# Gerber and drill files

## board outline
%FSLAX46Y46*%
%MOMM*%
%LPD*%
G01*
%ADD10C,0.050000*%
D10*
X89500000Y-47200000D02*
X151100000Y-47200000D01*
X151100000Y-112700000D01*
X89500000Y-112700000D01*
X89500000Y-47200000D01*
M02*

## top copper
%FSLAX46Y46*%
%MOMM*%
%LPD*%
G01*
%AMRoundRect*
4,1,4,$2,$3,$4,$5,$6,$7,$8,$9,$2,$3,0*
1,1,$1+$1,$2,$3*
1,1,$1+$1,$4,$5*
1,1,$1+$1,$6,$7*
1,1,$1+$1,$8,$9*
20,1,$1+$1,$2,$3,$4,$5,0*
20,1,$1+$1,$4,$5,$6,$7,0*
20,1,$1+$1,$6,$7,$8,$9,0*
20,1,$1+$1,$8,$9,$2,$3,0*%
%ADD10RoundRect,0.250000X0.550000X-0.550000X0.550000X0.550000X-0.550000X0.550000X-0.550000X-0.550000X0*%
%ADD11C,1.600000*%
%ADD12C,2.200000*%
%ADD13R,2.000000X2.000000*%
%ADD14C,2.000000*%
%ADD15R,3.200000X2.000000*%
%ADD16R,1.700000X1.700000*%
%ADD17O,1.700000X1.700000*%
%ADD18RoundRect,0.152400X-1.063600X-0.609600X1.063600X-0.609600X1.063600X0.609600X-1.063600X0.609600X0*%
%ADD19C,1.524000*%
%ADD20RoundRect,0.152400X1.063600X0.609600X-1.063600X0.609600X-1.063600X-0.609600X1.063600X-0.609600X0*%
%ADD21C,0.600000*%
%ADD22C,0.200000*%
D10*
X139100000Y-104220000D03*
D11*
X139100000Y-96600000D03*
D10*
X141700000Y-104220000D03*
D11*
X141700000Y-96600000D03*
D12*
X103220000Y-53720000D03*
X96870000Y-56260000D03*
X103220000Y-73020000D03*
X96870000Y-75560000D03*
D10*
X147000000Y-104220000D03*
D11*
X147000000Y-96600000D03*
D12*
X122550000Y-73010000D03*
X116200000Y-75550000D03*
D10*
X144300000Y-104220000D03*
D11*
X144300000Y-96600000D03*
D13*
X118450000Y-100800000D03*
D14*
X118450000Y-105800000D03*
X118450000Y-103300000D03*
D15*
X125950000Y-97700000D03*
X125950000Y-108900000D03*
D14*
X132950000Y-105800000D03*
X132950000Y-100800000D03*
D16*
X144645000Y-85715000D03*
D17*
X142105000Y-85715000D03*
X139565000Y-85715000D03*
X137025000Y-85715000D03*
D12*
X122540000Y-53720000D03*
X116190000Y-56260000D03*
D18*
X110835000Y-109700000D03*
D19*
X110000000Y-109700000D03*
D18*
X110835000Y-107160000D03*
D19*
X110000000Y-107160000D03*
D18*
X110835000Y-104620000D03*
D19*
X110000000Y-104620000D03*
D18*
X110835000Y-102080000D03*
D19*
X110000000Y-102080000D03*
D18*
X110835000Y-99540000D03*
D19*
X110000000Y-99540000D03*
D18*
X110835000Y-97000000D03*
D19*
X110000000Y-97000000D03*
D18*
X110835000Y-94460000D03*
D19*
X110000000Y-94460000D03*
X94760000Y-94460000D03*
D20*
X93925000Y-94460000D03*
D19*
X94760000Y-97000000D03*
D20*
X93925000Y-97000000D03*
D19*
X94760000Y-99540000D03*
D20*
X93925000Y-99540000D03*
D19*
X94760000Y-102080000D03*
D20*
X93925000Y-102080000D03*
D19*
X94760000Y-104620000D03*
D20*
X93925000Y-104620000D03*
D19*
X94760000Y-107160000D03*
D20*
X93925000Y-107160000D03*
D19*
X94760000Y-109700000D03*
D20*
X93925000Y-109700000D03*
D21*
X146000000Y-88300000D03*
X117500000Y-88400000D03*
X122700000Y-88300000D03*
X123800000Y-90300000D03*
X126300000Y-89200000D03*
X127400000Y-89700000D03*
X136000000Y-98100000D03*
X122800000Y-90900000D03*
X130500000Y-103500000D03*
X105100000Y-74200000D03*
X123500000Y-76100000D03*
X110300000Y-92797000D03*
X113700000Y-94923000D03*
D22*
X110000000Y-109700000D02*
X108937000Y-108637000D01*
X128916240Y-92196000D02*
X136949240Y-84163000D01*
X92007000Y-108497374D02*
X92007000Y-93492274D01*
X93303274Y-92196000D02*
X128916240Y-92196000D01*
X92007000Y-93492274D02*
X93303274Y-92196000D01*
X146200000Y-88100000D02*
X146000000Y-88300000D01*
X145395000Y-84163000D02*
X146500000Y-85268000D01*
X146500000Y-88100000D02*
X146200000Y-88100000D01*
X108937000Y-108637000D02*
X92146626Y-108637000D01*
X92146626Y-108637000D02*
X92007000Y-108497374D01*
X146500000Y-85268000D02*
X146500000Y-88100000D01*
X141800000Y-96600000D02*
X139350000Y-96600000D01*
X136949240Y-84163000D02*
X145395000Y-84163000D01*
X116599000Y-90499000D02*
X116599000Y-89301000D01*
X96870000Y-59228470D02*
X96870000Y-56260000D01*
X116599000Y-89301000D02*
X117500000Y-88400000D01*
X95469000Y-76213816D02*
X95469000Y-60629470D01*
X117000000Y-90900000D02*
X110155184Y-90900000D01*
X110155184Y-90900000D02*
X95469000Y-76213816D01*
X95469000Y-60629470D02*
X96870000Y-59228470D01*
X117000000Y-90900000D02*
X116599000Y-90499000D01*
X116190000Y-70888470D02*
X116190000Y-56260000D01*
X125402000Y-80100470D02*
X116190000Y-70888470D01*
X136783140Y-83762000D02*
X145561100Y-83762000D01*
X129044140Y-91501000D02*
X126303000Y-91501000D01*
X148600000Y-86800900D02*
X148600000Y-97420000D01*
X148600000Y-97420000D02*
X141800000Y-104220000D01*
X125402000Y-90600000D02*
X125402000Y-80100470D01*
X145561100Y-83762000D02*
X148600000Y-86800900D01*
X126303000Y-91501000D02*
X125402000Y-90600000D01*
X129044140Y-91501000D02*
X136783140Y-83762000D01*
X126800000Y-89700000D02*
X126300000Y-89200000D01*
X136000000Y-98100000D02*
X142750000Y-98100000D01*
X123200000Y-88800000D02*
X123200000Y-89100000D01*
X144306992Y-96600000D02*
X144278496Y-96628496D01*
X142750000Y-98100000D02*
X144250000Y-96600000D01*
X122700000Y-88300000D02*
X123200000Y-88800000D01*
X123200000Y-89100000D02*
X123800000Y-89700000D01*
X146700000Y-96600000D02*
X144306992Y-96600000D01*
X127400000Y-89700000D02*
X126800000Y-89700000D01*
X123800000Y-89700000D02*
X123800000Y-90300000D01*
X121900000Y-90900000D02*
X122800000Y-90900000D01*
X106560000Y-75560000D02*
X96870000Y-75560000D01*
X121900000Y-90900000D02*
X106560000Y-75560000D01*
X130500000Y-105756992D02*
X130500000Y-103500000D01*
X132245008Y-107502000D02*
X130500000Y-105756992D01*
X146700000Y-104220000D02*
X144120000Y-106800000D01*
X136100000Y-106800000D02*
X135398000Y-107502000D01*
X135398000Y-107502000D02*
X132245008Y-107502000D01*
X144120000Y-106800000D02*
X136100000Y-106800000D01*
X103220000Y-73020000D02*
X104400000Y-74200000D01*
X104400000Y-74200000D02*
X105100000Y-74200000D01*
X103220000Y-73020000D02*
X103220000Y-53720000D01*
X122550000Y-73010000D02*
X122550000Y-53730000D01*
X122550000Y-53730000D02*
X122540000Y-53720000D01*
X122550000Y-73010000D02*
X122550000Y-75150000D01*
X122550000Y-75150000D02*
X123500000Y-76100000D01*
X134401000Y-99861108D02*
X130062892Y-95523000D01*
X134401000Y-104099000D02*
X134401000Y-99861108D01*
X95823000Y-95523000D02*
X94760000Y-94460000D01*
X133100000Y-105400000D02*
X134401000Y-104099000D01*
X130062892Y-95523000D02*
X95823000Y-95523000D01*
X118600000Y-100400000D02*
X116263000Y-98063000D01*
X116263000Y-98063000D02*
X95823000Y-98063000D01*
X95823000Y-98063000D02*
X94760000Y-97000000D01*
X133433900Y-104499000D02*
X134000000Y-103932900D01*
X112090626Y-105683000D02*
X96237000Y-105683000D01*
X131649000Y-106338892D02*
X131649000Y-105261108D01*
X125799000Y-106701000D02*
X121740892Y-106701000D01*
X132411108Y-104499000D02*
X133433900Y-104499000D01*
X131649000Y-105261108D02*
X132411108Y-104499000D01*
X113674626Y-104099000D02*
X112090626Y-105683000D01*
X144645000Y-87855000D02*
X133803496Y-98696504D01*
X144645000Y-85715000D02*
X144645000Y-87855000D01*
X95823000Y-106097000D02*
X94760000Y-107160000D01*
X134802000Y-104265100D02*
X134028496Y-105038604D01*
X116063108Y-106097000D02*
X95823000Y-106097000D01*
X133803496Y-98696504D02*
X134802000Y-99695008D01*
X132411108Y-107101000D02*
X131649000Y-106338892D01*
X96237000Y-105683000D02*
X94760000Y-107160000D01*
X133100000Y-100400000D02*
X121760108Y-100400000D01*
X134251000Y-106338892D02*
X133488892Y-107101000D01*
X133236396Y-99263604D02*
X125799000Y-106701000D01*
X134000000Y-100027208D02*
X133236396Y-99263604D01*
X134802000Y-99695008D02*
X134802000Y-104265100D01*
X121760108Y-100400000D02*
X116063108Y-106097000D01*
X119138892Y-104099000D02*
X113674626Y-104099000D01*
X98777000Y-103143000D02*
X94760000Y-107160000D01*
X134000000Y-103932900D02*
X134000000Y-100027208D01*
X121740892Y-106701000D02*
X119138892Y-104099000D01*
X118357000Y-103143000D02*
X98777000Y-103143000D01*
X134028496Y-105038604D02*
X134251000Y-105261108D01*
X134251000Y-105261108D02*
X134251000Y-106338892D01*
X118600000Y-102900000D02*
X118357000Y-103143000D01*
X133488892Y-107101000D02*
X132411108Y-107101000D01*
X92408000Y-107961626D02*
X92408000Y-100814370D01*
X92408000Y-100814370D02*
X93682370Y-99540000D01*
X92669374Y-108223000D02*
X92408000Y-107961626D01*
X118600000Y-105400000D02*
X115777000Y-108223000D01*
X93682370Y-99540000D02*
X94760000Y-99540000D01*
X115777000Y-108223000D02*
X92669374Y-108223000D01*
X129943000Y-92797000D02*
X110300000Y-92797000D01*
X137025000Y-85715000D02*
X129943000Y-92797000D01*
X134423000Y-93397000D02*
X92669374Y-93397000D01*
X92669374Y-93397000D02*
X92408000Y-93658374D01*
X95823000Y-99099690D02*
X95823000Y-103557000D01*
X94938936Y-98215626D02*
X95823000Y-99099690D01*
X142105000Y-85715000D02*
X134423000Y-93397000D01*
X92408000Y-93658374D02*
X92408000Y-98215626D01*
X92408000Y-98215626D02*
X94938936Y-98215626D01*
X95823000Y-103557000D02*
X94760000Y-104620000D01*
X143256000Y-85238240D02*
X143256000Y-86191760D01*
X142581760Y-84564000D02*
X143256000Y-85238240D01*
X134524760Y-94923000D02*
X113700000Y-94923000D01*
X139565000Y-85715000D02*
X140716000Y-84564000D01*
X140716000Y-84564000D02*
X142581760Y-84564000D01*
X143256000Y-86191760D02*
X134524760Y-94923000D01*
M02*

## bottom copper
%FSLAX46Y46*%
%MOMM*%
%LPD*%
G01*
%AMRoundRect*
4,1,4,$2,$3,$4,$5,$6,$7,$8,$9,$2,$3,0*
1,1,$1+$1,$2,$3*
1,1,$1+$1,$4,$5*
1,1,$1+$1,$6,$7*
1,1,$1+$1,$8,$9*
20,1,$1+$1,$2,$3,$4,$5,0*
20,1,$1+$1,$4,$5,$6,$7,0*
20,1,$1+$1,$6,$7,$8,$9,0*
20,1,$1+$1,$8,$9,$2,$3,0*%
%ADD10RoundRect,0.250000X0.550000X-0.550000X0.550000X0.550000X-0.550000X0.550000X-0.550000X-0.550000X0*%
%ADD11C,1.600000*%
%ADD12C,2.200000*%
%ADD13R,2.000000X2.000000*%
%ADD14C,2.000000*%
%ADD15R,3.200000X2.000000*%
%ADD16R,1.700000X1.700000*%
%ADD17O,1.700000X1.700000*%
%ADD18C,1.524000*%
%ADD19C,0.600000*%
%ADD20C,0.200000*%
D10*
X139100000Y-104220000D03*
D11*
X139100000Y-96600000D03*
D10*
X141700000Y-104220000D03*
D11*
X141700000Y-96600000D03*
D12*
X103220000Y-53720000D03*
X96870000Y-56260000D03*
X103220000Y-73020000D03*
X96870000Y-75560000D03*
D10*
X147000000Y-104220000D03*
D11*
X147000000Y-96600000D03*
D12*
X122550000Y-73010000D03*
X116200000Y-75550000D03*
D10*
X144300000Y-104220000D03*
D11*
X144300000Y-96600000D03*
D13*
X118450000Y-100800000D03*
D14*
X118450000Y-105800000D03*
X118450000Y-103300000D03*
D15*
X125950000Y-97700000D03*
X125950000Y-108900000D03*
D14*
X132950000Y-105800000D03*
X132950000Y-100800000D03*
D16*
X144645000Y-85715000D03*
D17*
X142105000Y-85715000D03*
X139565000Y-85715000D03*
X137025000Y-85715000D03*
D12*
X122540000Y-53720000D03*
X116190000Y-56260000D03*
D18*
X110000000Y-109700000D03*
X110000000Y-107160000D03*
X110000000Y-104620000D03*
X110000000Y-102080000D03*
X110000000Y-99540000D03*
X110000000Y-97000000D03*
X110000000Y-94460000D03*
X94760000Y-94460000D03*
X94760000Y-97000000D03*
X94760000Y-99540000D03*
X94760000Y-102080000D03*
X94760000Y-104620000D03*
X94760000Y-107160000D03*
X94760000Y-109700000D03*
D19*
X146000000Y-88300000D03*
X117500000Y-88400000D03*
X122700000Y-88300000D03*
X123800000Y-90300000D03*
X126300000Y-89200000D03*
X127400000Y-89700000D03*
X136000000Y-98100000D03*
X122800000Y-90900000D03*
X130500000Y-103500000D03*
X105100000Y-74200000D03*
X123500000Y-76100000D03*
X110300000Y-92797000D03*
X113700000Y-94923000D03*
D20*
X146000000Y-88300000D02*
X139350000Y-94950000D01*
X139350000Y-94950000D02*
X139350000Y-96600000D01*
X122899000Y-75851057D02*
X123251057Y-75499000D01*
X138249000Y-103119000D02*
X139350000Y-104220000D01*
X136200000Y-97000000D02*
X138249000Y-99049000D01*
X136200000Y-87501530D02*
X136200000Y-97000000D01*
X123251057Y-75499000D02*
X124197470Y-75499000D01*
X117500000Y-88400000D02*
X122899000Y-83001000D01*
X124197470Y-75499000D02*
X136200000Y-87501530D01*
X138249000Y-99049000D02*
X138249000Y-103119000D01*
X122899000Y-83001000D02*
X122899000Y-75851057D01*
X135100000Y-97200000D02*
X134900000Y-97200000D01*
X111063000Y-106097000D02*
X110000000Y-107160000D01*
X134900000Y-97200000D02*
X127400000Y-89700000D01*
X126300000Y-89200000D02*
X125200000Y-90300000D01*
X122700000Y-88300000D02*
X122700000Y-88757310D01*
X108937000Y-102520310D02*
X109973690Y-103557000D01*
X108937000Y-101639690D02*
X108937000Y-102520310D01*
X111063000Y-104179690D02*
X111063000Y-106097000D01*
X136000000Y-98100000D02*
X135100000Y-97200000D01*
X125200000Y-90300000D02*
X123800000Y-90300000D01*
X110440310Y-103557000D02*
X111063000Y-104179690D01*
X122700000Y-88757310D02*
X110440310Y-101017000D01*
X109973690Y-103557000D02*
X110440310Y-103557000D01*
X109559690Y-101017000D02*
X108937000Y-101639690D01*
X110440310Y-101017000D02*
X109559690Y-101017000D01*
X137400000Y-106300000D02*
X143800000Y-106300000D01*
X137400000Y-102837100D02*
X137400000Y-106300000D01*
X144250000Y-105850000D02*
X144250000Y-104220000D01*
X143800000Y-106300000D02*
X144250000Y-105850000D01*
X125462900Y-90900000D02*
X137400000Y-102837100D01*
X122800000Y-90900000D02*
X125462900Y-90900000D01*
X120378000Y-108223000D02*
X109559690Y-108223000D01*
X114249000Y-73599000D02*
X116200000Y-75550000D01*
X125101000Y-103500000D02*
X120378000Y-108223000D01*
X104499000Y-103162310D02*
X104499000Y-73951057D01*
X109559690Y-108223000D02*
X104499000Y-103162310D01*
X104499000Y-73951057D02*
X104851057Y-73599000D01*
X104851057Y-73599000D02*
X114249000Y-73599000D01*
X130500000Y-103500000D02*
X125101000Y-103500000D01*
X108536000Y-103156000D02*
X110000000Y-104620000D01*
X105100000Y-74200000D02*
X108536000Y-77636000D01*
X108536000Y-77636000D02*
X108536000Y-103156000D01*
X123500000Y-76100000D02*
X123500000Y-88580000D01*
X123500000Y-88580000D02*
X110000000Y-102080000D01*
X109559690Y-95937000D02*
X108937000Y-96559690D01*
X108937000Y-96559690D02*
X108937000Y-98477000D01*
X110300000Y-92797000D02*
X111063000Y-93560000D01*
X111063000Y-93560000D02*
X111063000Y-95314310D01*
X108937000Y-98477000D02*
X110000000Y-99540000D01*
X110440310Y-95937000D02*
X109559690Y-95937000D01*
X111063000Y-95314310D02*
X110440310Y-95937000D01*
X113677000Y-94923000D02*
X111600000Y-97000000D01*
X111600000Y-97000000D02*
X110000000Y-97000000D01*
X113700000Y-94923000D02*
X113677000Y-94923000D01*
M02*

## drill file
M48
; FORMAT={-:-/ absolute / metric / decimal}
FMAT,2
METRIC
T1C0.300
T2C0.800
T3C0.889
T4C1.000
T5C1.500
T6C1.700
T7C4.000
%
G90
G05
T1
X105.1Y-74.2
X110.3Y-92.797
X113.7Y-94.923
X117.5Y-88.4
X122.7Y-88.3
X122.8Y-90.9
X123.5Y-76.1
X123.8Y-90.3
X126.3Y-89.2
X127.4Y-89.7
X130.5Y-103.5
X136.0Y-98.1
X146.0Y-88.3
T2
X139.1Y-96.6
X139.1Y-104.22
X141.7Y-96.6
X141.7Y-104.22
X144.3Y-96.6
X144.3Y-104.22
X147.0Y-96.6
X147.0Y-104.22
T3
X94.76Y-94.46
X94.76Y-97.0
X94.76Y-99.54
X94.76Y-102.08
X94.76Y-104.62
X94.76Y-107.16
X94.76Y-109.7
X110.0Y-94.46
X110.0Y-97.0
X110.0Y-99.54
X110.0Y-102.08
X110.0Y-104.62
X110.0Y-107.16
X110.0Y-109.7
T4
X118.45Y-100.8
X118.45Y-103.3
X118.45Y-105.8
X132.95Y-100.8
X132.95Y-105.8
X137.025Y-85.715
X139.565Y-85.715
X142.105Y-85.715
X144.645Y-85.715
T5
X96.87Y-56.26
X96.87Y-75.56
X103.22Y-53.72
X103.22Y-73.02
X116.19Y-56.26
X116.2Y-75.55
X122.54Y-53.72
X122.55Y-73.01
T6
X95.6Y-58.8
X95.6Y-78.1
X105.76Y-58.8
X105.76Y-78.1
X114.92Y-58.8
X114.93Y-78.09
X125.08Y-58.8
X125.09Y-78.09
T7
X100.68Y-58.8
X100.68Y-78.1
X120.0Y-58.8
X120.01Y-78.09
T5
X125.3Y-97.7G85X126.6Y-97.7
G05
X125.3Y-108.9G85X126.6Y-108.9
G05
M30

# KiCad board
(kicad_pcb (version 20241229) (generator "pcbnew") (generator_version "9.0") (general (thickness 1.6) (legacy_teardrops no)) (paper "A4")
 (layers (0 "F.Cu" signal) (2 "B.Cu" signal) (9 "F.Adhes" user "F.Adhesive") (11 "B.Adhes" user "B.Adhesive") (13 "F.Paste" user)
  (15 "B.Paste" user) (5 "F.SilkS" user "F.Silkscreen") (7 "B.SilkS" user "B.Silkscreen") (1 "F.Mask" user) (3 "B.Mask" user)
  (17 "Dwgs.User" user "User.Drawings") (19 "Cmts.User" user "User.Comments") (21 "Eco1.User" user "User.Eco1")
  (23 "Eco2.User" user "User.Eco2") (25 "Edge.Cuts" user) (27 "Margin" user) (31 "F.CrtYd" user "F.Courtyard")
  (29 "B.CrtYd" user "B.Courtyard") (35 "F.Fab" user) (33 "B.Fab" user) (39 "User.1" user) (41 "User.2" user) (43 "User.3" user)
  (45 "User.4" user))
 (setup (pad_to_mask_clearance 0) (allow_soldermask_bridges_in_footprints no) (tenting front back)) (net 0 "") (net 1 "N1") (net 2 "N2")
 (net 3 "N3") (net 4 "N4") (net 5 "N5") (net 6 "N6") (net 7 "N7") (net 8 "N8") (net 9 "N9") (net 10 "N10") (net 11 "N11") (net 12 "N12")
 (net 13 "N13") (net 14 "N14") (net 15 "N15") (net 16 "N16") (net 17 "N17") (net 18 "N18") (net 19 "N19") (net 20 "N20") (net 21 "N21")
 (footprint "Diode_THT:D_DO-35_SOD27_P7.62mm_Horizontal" (layer "F.Cu") (at 139.1 104.22 90)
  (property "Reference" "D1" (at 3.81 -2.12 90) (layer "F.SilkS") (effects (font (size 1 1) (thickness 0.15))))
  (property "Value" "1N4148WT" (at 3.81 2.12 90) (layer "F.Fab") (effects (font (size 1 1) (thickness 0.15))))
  (pad "1" thru_hole roundrect (at 0 0 90) (size 1.6 1.6) (drill 0.8) (layers "*.Cu" "*.Mask") (remove_unused_layers no)
   (roundrect_rratio 0.15625) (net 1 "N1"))
  (pad "2" thru_hole circle (at 7.62 0 90) (size 1.6 1.6) (drill 0.8) (layers "*.Cu" "*.Mask") (remove_unused_layers no) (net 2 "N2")))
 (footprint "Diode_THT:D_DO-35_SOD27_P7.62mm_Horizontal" (layer "F.Cu") (at 141.7 104.22 90)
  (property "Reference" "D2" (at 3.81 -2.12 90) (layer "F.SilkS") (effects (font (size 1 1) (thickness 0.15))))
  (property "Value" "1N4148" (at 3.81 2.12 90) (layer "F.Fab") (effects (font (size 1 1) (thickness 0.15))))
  (pad "1" thru_hole roundrect (at 0 0 90) (size 1.6 1.6) (drill 0.8) (layers "*.Cu" "*.Mask") (remove_unused_layers no)
   (roundrect_rratio 0.15625) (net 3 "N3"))
  (pad "2" thru_hole circle (at 7.62 0 90) (size 1.6 1.6) (drill 0.8) (layers "*.Cu" "*.Mask") (remove_unused_layers no) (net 2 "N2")))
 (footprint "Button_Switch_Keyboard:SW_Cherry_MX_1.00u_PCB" (layer "F.Cu") (at 103.22 53.72)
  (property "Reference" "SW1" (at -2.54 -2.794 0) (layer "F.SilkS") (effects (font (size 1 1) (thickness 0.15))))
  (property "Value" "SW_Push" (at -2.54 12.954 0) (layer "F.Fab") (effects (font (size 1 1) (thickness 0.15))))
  (pad "" np_thru_hole circle (at -7.62 5.08) (size 1.7 1.7) (drill 1.7) (layers "*.Cu" "*.Mask"))
  (pad "" np_thru_hole circle (at -2.54 5.08) (size 4 4) (drill 4) (layers "*.Cu" "*.Mask"))
  (pad "" np_thru_hole circle (at 2.54 5.08) (size 1.7 1.7) (drill 1.7) (layers "*.Cu" "*.Mask"))
  (pad "1" thru_hole circle (at 0 0) (size 2.2 2.2) (drill 1.5) (layers "*.Cu" "*.Mask") (remove_unused_layers no) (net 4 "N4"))
  (pad "2" thru_hole circle (at -6.35 2.54) (size 2.2 2.2) (drill 1.5) (layers "*.Cu" "*.Mask") (remove_unused_layers no) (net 1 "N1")))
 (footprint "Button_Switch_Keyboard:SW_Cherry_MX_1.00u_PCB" (layer "F.Cu") (at 103.22 73.02)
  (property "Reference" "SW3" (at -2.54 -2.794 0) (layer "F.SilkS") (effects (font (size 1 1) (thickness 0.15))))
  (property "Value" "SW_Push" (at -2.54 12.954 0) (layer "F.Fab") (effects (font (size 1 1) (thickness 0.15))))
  (pad "" np_thru_hole circle (at -7.62 5.08) (size 1.7 1.7) (drill 1.7) (layers "*.Cu" "*.Mask"))
  (pad "" np_thru_hole circle (at -2.54 5.08) (size 4 4) (drill 4) (layers "*.Cu" "*.Mask"))
  (pad "" np_thru_hole circle (at 2.54 5.08) (size 1.7 1.7) (drill 1.7) (layers "*.Cu" "*.Mask"))
  (pad "1" thru_hole circle (at 0 0) (size 2.2 2.2) (drill 1.5) (layers "*.Cu" "*.Mask") (remove_unused_layers no) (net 4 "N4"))
  (pad "2" thru_hole circle (at -6.35 2.54) (size 2.2 2.2) (drill 1.5) (layers "*.Cu" "*.Mask") (remove_unused_layers no) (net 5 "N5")))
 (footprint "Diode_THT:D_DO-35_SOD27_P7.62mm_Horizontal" (layer "F.Cu") (at 147 104.22 90)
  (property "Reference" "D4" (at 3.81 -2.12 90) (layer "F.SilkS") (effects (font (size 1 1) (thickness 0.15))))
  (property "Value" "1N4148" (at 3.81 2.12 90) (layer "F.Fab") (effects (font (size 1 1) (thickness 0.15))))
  (pad "1" thru_hole roundrect (at 0 0 90) (size 1.6 1.6) (drill 0.8) (layers "*.Cu" "*.Mask") (remove_unused_layers no)
   (roundrect_rratio 0.15625) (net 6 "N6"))
  (pad "2" thru_hole circle (at 7.62 0 90) (size 1.6 1.6) (drill 0.8) (layers "*.Cu" "*.Mask") (remove_unused_layers no) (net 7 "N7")))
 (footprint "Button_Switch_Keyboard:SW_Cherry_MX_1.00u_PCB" (layer "F.Cu") (at 122.55 73.01)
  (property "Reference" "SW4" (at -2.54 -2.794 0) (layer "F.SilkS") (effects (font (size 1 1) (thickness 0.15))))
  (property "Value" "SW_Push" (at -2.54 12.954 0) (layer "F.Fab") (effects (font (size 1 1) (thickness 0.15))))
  (pad "" np_thru_hole circle (at -7.62 5.08) (size 1.7 1.7) (drill 1.7) (layers "*.Cu" "*.Mask"))
  (pad "" np_thru_hole circle (at -2.54 5.08) (size 4 4) (drill 4) (layers "*.Cu" "*.Mask"))
  (pad "" np_thru_hole circle (at 2.54 5.08) (size 1.7 1.7) (drill 1.7) (layers "*.Cu" "*.Mask"))
  (pad "1" thru_hole circle (at 0 0) (size 2.2 2.2) (drill 1.5) (layers "*.Cu" "*.Mask") (remove_unused_layers no) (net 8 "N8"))
  (pad "2" thru_hole circle (at -6.35 2.54) (size 2.2 2.2) (drill 1.5) (layers "*.Cu" "*.Mask") (remove_unused_layers no) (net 6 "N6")))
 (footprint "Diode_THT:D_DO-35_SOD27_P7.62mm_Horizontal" (layer "F.Cu") (at 144.3 104.22 90)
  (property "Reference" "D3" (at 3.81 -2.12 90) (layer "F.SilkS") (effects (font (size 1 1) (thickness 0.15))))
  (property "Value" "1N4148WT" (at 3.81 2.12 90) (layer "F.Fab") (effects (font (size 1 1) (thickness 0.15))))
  (pad "1" thru_hole roundrect (at 0 0 90) (size 1.6 1.6) (drill 0.8) (layers "*.Cu" "*.Mask") (remove_unused_layers no)
   (roundrect_rratio 0.15625) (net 5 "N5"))
  (pad "2" thru_hole circle (at 7.62 0 90) (size 1.6 1.6) (drill 0.8) (layers "*.Cu" "*.Mask") (remove_unused_layers no) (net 7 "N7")))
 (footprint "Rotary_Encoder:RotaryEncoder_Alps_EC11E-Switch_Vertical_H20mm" (layer "F.Cu") (at 118.45 100.8)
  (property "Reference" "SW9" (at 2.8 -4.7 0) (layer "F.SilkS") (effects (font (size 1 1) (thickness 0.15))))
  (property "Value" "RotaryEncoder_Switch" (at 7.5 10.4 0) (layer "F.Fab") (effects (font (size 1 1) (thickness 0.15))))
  (pad "A" thru_hole rect (at 0 0) (size 2 2) (drill 1) (layers "*.Cu" "*.Mask") (remove_unused_layers no) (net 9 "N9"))
  (pad "B" thru_hole circle (at 0 5) (size 2 2) (drill 1) (layers "*.Cu" "*.Mask") (remove_unused_layers no) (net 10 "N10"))
  (pad "C" thru_hole circle (at 0 2.5) (size 2 2) (drill 1) (layers "*.Cu" "*.Mask") (remove_unused_layers no) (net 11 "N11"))
  (pad "MP" thru_hole rect (at 7.5 -3.1) (size 3.2 2) (drill oval 2.8 1.5) (layers "*.Cu" "*.Mask") (remove_unused_layers no))
  (pad "MP" thru_hole rect (at 7.5 8.1) (size 3.2 2) (drill oval 2.8 1.5) (layers "*.Cu" "*.Mask") (remove_unused_layers no))
  (pad "S1" thru_hole circle (at 14.5 5) (size 2 2) (drill 1) (layers "*.Cu" "*.Mask") (remove_unused_layers no) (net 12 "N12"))
  (pad "S2" thru_hole circle (at 14.5 0) (size 2 2) (drill 1) (layers "*.Cu" "*.Mask") (remove_unused_layers no) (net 11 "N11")))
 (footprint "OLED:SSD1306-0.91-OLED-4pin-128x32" (layer "F.Cu") (at 146.835 49.215 -90)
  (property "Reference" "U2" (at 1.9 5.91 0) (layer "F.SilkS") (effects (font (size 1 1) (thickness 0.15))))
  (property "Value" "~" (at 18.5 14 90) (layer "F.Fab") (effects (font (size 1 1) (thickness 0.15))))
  (pad "1" thru_hole rect (at 36.5 2.19 270) (size 1.7 1.7) (drill 1) (layers "*.Cu" "*.Mask") (remove_unused_layers no) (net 11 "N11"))
  (pad "2" thru_hole oval (at 36.5 4.73 270) (size 1.7 1.7) (drill 1) (layers "*.Cu" "*.Mask") (remove_unused_layers no) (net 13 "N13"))
  (pad "3" thru_hole oval (at 36.5 7.27 270) (size 1.7 1.7) (drill 1) (layers "*.Cu" "*.Mask") (remove_unused_layers no) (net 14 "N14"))
  (pad "4" thru_hole oval (at 36.5 9.81 270) (size 1.7 1.7) (drill 1) (layers "*.Cu" "*.Mask") (remove_unused_layers no) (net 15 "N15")))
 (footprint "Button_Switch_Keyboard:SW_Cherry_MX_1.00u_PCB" (layer "F.Cu") (at 122.54 53.72)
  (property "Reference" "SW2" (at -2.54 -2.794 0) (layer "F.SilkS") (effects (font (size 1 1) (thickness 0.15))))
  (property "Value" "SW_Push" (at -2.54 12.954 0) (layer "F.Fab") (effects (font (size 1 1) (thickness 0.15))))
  (pad "" np_thru_hole circle (at -7.62 5.08) (size 1.7 1.7) (drill 1.7) (layers "*.Cu" "*.Mask"))
  (pad "" np_thru_hole circle (at -2.54 5.08) (size 4 4) (drill 4) (layers "*.Cu" "*.Mask"))
  (pad "" np_thru_hole circle (at 2.54 5.08) (size 1.7 1.7) (drill 1.7) (layers "*.Cu" "*.Mask"))
  (pad "1" thru_hole circle (at 0 0) (size 2.2 2.2) (drill 1.5) (layers "*.Cu" "*.Mask") (remove_unused_layers no) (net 8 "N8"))
  (pad "2" thru_hole circle (at -6.35 2.54) (size 2.2 2.2) (drill 1.5) (layers "*.Cu" "*.Mask") (remove_unused_layers no) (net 3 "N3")))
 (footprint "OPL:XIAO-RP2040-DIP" (layer "F.Cu") (at 102.38 102.08 180)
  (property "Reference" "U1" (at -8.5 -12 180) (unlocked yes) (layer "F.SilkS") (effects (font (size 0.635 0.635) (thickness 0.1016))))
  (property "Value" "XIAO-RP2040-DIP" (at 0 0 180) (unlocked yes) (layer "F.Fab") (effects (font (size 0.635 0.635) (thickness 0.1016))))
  (pad "1" smd roundrect (at -8.455 -7.62) (size 2.432 1.524) (layers "F.Cu" "F.Mask") (roundrect_rratio 0.1) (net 2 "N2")
   (thermal_bridge_angle 45))
  (pad "1" thru_hole circle (at -7.62 -7.62) (size 1.524 1.524) (drill 0.889) (layers "*.Cu" "*.Mask") (remove_unused_layers no)
   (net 2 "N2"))
  (pad "2" smd roundrect (at -8.455 -5.08) (size 2.432 1.524) (layers "F.Cu" "F.Mask") (roundrect_rratio 0.1) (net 7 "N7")
   (thermal_bridge_angle 45))
  (pad "2" thru_hole circle (at -7.62 -5.08) (size 1.524 1.524) (drill 0.889) (layers "*.Cu" "*.Mask") (remove_unused_layers no)
   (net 7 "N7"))
  (pad "3" smd roundrect (at -8.455 -2.54) (size 2.432 1.524) (layers "F.Cu" "F.Mask") (roundrect_rratio 0.1) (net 4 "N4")
   (thermal_bridge_angle 45))
  (pad "3" thru_hole circle (at -7.62 -2.54) (size 1.524 1.524) (drill 0.889) (layers "*.Cu" "*.Mask") (remove_unused_layers no)
   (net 4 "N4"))
  (pad "4" smd roundrect (at -8.455 0) (size 2.432 1.524) (layers "F.Cu" "F.Mask") (roundrect_rratio 0.1) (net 8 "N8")
   (thermal_bridge_angle 45))
  (pad "4" thru_hole circle (at -7.62 0) (size 1.524 1.524) (drill 0.889) (layers "*.Cu" "*.Mask") (remove_unused_layers no) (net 8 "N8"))
  (pad "5" smd roundrect (at -8.455 2.54) (size 2.432 1.524) (layers "F.Cu" "F.Mask") (roundrect_rratio 0.1) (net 15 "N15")
   (thermal_bridge_angle 45))
  (pad "5" thru_hole circle (at -7.62 2.54) (size 1.524 1.524) (drill 0.889) (layers "*.Cu" "*.Mask") (remove_unused_layers no)
   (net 15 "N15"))
  (pad "6" smd roundrect (at -8.455 5.08) (size 2.432 1.524) (layers "F.Cu" "F.Mask") (roundrect_rratio 0.1) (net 14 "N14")
   (thermal_bridge_angle 45))
  (pad "6" thru_hole circle (at -7.62 5.08) (size 1.524 1.524) (drill 0.889) (layers "*.Cu" "*.Mask") (remove_unused_layers no)
   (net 14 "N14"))
  (pad "7" smd roundrect (at -8.455 7.62) (size 2.432 1.524) (layers "F.Cu" "F.Mask") (roundrect_rratio 0.1) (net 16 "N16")
   (thermal_bridge_angle 45))
  (pad "7" thru_hole circle (at -7.62 7.62) (size 1.524 1.524) (drill 0.889) (layers "*.Cu" "*.Mask") (remove_unused_layers no)
   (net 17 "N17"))
  (pad "8" thru_hole circle (at 7.62 7.62 180) (size 1.524 1.524) (drill 0.889) (layers "*.Cu" "*.Mask") (remove_unused_layers no)
   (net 12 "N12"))
  (pad "8" smd roundrect (at 8.455 7.62 180) (size 2.432 1.524) (layers "F.Cu" "F.Mask") (roundrect_rratio 0.1) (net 12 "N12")
   (thermal_bridge_angle 45))
  (pad "9" thru_hole circle (at 7.62 5.08 180) (size 1.524 1.524) (drill 0.889) (layers "*.Cu" "*.Mask") (remove_unused_layers no)
   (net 9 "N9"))
  (pad "9" smd roundrect (at 8.455 5.08 180) (size 2.432 1.524) (layers "F.Cu" "F.Mask") (roundrect_rratio 0.1) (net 9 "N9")
   (thermal_bridge_angle 45))
  (pad "10" thru_hole circle (at 7.62 2.54 180) (size 1.524 1.524) (drill 0.889) (layers "*.Cu" "*.Mask") (remove_unused_layers no)
   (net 10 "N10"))
  (pad "10" smd roundrect (at 8.455 2.54 180) (size 2.432 1.524) (layers "F.Cu" "F.Mask") (roundrect_rratio 0.1) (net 10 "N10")
   (thermal_bridge_angle 45))
  (pad "11" thru_hole circle (at 7.62 0 180) (size 1.524 1.524) (drill 0.889) (layers "*.Cu" "*.Mask") (remove_unused_layers no)
   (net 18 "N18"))
  (pad "11" smd roundrect (at 8.455 0 180) (size 2.432 1.524) (layers "F.Cu" "F.Mask") (roundrect_rratio 0.1) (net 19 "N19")
   (thermal_bridge_angle 45))
  (pad "12" thru_hole circle (at 7.62 -2.54 180) (size 1.524 1.524) (drill 0.889) (layers "*.Cu" "*.Mask") (remove_unused_layers no)
   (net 13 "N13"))
  (pad "12" smd roundrect (at 8.455 -2.54 180) (size 2.432 1.524) (layers "F.Cu" "F.Mask") (roundrect_rratio 0.1) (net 13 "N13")
   (thermal_bridge_angle 45))
  (pad "13" thru_hole circle (at 7.62 -5.08 180) (size 1.524 1.524) (drill 0.889) (layers "*.Cu" "*.Mask") (remove_unused_layers no)
   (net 11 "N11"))
  (pad "13" smd roundrect (at 8.455 -5.08 180) (size 2.432 1.524) (layers "F.Cu" "F.Mask") (roundrect_rratio 0.1) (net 11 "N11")
   (thermal_bridge_angle 45))
  (pad "14" thru_hole circle (at 7.62 -7.62 180) (size 1.524 1.524) (drill 0.889) (layers "*.Cu" "*.Mask") (remove_unused_layers no)
   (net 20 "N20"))
  (pad "14" smd roundrect (at 8.455 -7.62 180) (size 2.432 1.524) (layers "F.Cu" "F.Mask") (roundrect_rratio 0.1) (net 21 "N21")
   (thermal_bridge_angle 45)))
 (gr_rect (start 89.5 47.2) (end 151.1 112.7) (stroke (width 0.05) (type default)) (fill no) (layer "Edge.Cuts"))
 (segment (start 110 109.7) (end 108.937 108.637) (width 0.2) (layer "F.Cu") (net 2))
 (segment (start 128.91624 92.196) (end 136.94924 84.163) (width 0.2) (layer "F.Cu") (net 2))
 (segment (start 92.007 108.497374) (end 92.007 93.492274) (width 0.2) (layer "F.Cu") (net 2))
 (segment (start 93.303274 92.196) (end 128.91624 92.196) (width 0.2) (layer "F.Cu") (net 2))
 (segment (start 92.007 93.492274) (end 93.303274 92.196) (width 0.2) (layer "F.Cu") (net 2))
 (segment (start 146.2 88.1) (end 146 88.3) (width 0.2) (layer "F.Cu") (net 2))
 (segment (start 145.395 84.163) (end 146.5 85.268) (width 0.2) (layer "F.Cu") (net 2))
 (segment (start 146.5 88.1) (end 146.2 88.1) (width 0.2) (layer "F.Cu") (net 2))
 (segment (start 108.937 108.637) (end 92.146626 108.637) (width 0.2) (layer "F.Cu") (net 2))
 (segment (start 92.146626 108.637) (end 92.007 108.497374) (width 0.2) (layer "F.Cu") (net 2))
 (segment (start 146.5 85.268) (end 146.5 88.1) (width 0.2) (layer "F.Cu") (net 2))
 (segment (start 141.8 96.6) (end 139.35 96.6) (width 0.2) (layer "F.Cu") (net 2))
 (segment (start 136.94924 84.163) (end 145.395 84.163) (width 0.2) (layer "F.Cu") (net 2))
 (via (at 146 88.3) (size 0.6) (drill 0.3) (layers "F.Cu" "B.Cu") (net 2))
 (segment (start 146 88.3) (end 139.35 94.95) (width 0.2) (layer "B.Cu") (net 2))
 (segment (start 139.35 94.95) (end 139.35 96.6) (width 0.2) (layer "B.Cu") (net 2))
 (segment (start 116.599 90.499) (end 116.599 89.301) (width 0.2) (layer "F.Cu") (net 1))
 (segment (start 96.87 59.22847) (end 96.87 56.26) (width 0.2) (layer "F.Cu") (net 1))
 (segment (start 116.599 89.301) (end 117.5 88.4) (width 0.2) (layer "F.Cu") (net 1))
 (segment (start 95.469 76.213816) (end 95.469 60.62947) (width 0.2) (layer "F.Cu") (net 1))
 (segment (start 117 90.9) (end 110.155184 90.9) (width 0.2) (layer "F.Cu") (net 1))
 (segment (start 110.155184 90.9) (end 95.469 76.213816) (width 0.2) (layer "F.Cu") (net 1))
 (segment (start 95.469 60.62947) (end 96.87 59.22847) (width 0.2) (layer "F.Cu") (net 1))
 (segment (start 117 90.9) (end 116.599 90.499) (width 0.2) (layer "F.Cu") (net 1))
 (via (at 117.5 88.4) (size 0.6) (drill 0.3) (layers "F.Cu" "B.Cu") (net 1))
 (segment (start 122.899 75.851057) (end 123.251057 75.499) (width 0.2) (layer "B.Cu") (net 1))
 (segment (start 138.249 103.119) (end 139.35 104.22) (width 0.2) (layer "B.Cu") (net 1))
 (segment (start 136.2 97) (end 138.249 99.049) (width 0.2) (layer "B.Cu") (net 1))
 (segment (start 136.2 87.50153) (end 136.2 97) (width 0.2) (layer "B.Cu") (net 1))
 (segment (start 123.251057 75.499) (end 124.19747 75.499) (width 0.2) (layer "B.Cu") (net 1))
 (segment (start 117.5 88.4) (end 122.899 83.001) (width 0.2) (layer "B.Cu") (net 1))
 (segment (start 124.19747 75.499) (end 136.2 87.50153) (width 0.2) (layer "B.Cu") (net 1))
 (segment (start 138.249 99.049) (end 138.249 103.119) (width 0.2) (layer "B.Cu") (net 1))
 (segment (start 122.899 83.001) (end 122.899 75.851057) (width 0.2) (layer "B.Cu") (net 1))
 (segment (start 116.19 70.88847) (end 116.19 56.26) (width 0.2) (layer "F.Cu") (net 3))
 (segment (start 125.402 80.10047) (end 116.19 70.88847) (width 0.2) (layer "F.Cu") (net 3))
 (segment (start 136.78314 83.762) (end 145.5611 83.762) (width 0.2) (layer "F.Cu") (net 3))
 (segment (start 129.04414 91.501) (end 126.303 91.501) (width 0.2) (layer "F.Cu") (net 3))
 (segment (start 148.6 86.8009) (end 148.6 97.42) (width 0.2) (layer "F.Cu") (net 3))
 (segment (start 148.6 97.42) (end 141.8 104.22) (width 0.2) (layer "F.Cu") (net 3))
 (segment (start 125.402 90.6) (end 125.402 80.10047) (width 0.2) (layer "F.Cu") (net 3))
 (segment (start 145.5611 83.762) (end 148.6 86.8009) (width 0.2) (layer "F.Cu") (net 3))
 (segment (start 126.303 91.501) (end 125.402 90.6) (width 0.2) (layer "F.Cu") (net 3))
 (segment (start 129.04414 91.501) (end 136.78314 83.762) (width 0.2) (layer "F.Cu") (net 3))
 (segment (start 126.8 89.7) (end 126.3 89.2) (width 0.2) (layer "F.Cu") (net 7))
 (segment (start 136 98.1) (end 142.75 98.1) (width 0.2) (layer "F.Cu") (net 7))
 (segment (start 123.2 88.8) (end 123.2 89.1) (width 0.2) (layer "F.Cu") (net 7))
 (segment (start 144.306992 96.6) (end 144.278496 96.628496) (width 0.2) (layer "F.Cu") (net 7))
 (segment (start 142.75 98.1) (end 144.25 96.6) (width 0.2) (layer "F.Cu") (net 7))
 (segment (start 122.7 88.3) (end 123.2 88.8) (width 0.2) (layer "F.Cu") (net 7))
 (segment (start 123.2 89.1) (end 123.8 89.7) (width 0.2) (layer "F.Cu") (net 7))
 (segment (start 146.7 96.6) (end 144.306992 96.6) (width 0.2) (layer "F.Cu") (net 7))
 (segment (start 127.4 89.7) (end 126.8 89.7) (width 0.2) (layer "F.Cu") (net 7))
 (segment (start 123.8 89.7) (end 123.8 90.3) (width 0.2) (layer "F.Cu") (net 7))
 (via (at 122.7 88.3) (size 0.6) (drill 0.3) (layers "F.Cu" "B.Cu") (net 7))
 (via (at 123.8 90.3) (size 0.6) (drill 0.3) (layers "F.Cu" "B.Cu") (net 7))
 (via (at 126.3 89.2) (size 0.6) (drill 0.3) (layers "F.Cu" "B.Cu") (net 7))
 (via (at 127.4 89.7) (size 0.6) (drill 0.3) (layers "F.Cu" "B.Cu") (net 7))
 (via (at 136 98.1) (size 0.6) (drill 0.3) (layers "F.Cu" "B.Cu") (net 7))
 (segment (start 135.1 97.2) (end 134.9 97.2) (width 0.2) (layer "B.Cu") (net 7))
 (segment (start 111.063 106.097) (end 110 107.16) (width 0.2) (layer "B.Cu") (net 7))
 (segment (start 134.9 97.2) (end 127.4 89.7) (width 0.2) (layer "B.Cu") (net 7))
 (segment (start 126.3 89.2) (end 125.2 90.3) (width 0.2) (layer "B.Cu") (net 7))
 (segment (start 122.7 88.3) (end 122.7 88.75731) (width 0.2) (layer "B.Cu") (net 7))
 (segment (start 108.937 102.52031) (end 109.97369 103.557) (width 0.2) (layer "B.Cu") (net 7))
 (segment (start 108.937 101.63969) (end 108.937 102.52031) (width 0.2) (layer "B.Cu") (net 7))
 (segment (start 111.063 104.17969) (end 111.063 106.097) (width 0.2) (layer "B.Cu") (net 7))
 (segment (start 136 98.1) (end 135.1 97.2) (width 0.2) (layer "B.Cu") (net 7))
 (segment (start 125.2 90.3) (end 123.8 90.3) (width 0.2) (layer "B.Cu") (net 7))
 (segment (start 110.44031 103.557) (end 111.063 104.17969) (width 0.2) (layer "B.Cu") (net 7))
 (segment (start 122.7 88.75731) (end 110.44031 101.017) (width 0.2) (layer "B.Cu") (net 7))
 (segment (start 109.97369 103.557) (end 110.44031 103.557) (width 0.2) (layer "B.Cu") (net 7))
 (segment (start 109.55969 101.017) (end 108.937 101.63969) (width 0.2) (layer "B.Cu") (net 7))
 (segment (start 110.44031 101.017) (end 109.55969 101.017) (width 0.2) (layer "B.Cu") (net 7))
 (segment (start 121.9 90.9) (end 122.8 90.9) (width 0.2) (layer "F.Cu") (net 5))
 (segment (start 106.56 75.56) (end 96.87 75.56) (width 0.2) (layer "F.Cu") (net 5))
 (segment (start 121.9 90.9) (end 106.56 75.56) (width 0.2) (layer "F.Cu") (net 5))
 (via (at 122.8 90.9) (size 0.6) (drill 0.3) (layers "F.Cu" "B.Cu") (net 5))
 (segment (start 137.4 106.3) (end 143.8 106.3) (width 0.2) (layer "B.Cu") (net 5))
 (segment (start 137.4 102.8371) (end 137.4 106.3) (width 0.2) (layer "B.Cu") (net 5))
 (segment (start 144.25 105.85) (end 144.25 104.22) (width 0.2) (layer "B.Cu") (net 5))
 (segment (start 143.8 106.3) (end 144.25 105.85) (width 0.2) (layer "B.Cu") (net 5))
 (segment (start 125.4629 90.9) (end 137.4 102.8371) (width 0.2) (layer "B.Cu") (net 5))
 (segment (start 122.8 90.9) (end 125.4629 90.9) (width 0.2) (layer "B.Cu") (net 5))
 (segment (start 130.5 105.756992) (end 130.5 103.5) (width 0.2) (layer "F.Cu") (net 6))
 (segment (start 132.245008 107.502) (end 130.5 105.756992) (width 0.2) (layer "F.Cu") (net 6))
 (segment (start 146.7 104.22) (end 144.12 106.8) (width 0.2) (layer "F.Cu") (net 6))
 (segment (start 136.1 106.8) (end 135.398 107.502) (width 0.2) (layer "F.Cu") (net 6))
 (segment (start 135.398 107.502) (end 132.245008 107.502) (width 0.2) (layer "F.Cu") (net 6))
 (segment (start 144.12 106.8) (end 136.1 106.8) (width 0.2) (layer "F.Cu") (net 6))
 (via (at 130.5 103.5) (size 0.6) (drill 0.3) (layers "F.Cu" "B.Cu") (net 6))
 (segment (start 120.378 108.223) (end 109.55969 108.223) (width 0.2) (layer "B.Cu") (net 6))
 (segment (start 114.249 73.599) (end 116.2 75.55) (width 0.2) (layer "B.Cu") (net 6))
 (segment (start 125.101 103.5) (end 120.378 108.223) (width 0.2) (layer "B.Cu") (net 6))
 (segment (start 104.499 103.16231) (end 104.499 73.951057) (width 0.2) (layer "B.Cu") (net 6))
 (segment (start 109.55969 108.223) (end 104.499 103.16231) (width 0.2) (layer "B.Cu") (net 6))
 (segment (start 104.499 73.951057) (end 104.851057 73.599) (width 0.2) (layer "B.Cu") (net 6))
 (segment (start 104.851057 73.599) (end 114.249 73.599) (width 0.2) (layer "B.Cu") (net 6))
 (segment (start 130.5 103.5) (end 125.101 103.5) (width 0.2) (layer "B.Cu") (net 6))
 (segment (start 103.22 73.02) (end 104.4 74.2) (width 0.2) (layer "F.Cu") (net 4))
 (segment (start 104.4 74.2) (end 105.1 74.2) (width 0.2) (layer "F.Cu") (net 4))
 (segment (start 103.22 73.02) (end 103.22 53.72) (width 0.2) (layer "F.Cu") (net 4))
 (via (at 105.1 74.2) (size 0.6) (drill 0.3) (layers "F.Cu" "B.Cu") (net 4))
 (segment (start 108.536 103.156) (end 110 104.62) (width 0.2) (layer "B.Cu") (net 4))
 (segment (start 105.1 74.2) (end 108.536 77.636) (width 0.2) (layer "B.Cu") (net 4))
 (segment (start 108.536 77.636) (end 108.536 103.156) (width 0.2) (layer "B.Cu") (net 4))
 (segment (start 122.55 73.01) (end 122.55 53.73) (width 0.2) (layer "F.Cu") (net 8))
 (segment (start 122.55 53.73) (end 122.54 53.72) (width 0.2) (layer "F.Cu") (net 8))
 (segment (start 122.55 73.01) (end 122.55 75.15) (width 0.2) (layer "F.Cu") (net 8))
 (segment (start 122.55 75.15) (end 123.5 76.1) (width 0.2) (layer "F.Cu") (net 8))
 (via (at 123.5 76.1) (size 0.6) (drill 0.3) (layers "F.Cu" "B.Cu") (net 8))
 (segment (start 123.5 76.1) (end 123.5 88.58) (width 0.2) (layer "B.Cu") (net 8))
 (segment (start 123.5 88.58) (end 110 102.08) (width 0.2) (layer "B.Cu") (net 8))
 (segment (start 134.401 99.861108) (end 130.062892 95.523) (width 0.2) (layer "F.Cu") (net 12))
 (segment (start 134.401 104.099) (end 134.401 99.861108) (width 0.2) (layer "F.Cu") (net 12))
 (segment (start 95.823 95.523) (end 94.76 94.46) (width 0.2) (layer "F.Cu") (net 12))
 (segment (start 133.1 105.4) (end 134.401 104.099) (width 0.2) (layer "F.Cu") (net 12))
 (segment (start 130.062892 95.523) (end 95.823 95.523) (width 0.2) (layer "F.Cu") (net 12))
 (segment (start 118.6 100.4) (end 116.263 98.063) (width 0.2) (layer "F.Cu") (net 9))
 (segment (start 116.263 98.063) (end 95.823 98.063) (width 0.2) (layer "F.Cu") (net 9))
 (segment (start 95.823 98.063) (end 94.76 97) (width 0.2) (layer "F.Cu") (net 9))
 (segment (start 133.4339 104.499) (end 134 103.9329) (width 0.2) (layer "F.Cu") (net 11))
 (segment (start 112.090626 105.683) (end 96.237 105.683) (width 0.2) (layer "F.Cu") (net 11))
 (segment (start 131.649 106.338892) (end 131.649 105.261108) (width 0.2) (layer "F.Cu") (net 11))
 (segment (start 125.799 106.701) (end 121.740892 106.701) (width 0.2) (layer "F.Cu") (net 11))
 (segment (start 132.411108 104.499) (end 133.4339 104.499) (width 0.2) (layer "F.Cu") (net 11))
 (segment (start 131.649 105.261108) (end 132.411108 104.499) (width 0.2) (layer "F.Cu") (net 11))
 (segment (start 113.674626 104.099) (end 112.090626 105.683) (width 0.2) (layer "F.Cu") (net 11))
 (segment (start 144.645 87.855) (end 133.803496 98.696504) (width 0.2) (layer "F.Cu") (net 11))
 (segment (start 144.645 85.715) (end 144.645 87.855) (width 0.2) (layer "F.Cu") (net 11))
 (segment (start 95.823 106.097) (end 94.76 107.16) (width 0.2) (layer "F.Cu") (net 11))
 (segment (start 134.802 104.2651) (end 134.028496 105.038604) (width 0.2) (layer "F.Cu") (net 11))
 (segment (start 116.063108 106.097) (end 95.823 106.097) (width 0.2) (layer "F.Cu") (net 11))
 (segment (start 133.803496 98.696504) (end 134.802 99.695008) (width 0.2) (layer "F.Cu") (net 11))
 (segment (start 132.411108 107.101) (end 131.649 106.338892) (width 0.2) (layer "F.Cu") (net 11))
 (segment (start 96.237 105.683) (end 94.76 107.16) (width 0.2) (layer "F.Cu") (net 11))
 (segment (start 133.1 100.4) (end 121.760108 100.4) (width 0.2) (layer "F.Cu") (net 11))
 (segment (start 134.251 106.338892) (end 133.488892 107.101) (width 0.2) (layer "F.Cu") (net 11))
 (segment (start 133.236396 99.263604) (end 125.799 106.701) (width 0.2) (layer "F.Cu") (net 11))
 (segment (start 134 100.027208) (end 133.236396 99.263604) (width 0.2) (layer "F.Cu") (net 11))
 (segment (start 134.802 99.695008) (end 134.802 104.2651) (width 0.2) (layer "F.Cu") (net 11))
 (segment (start 121.760108 100.4) (end 116.063108 106.097) (width 0.2) (layer "F.Cu") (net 11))
 (segment (start 119.138892 104.099) (end 113.674626 104.099) (width 0.2) (layer "F.Cu") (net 11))
 (segment (start 98.777 103.143) (end 94.76 107.16) (width 0.2) (layer "F.Cu") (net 11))
 (segment (start 134 103.9329) (end 134 100.027208) (width 0.2) (layer "F.Cu") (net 11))
 (segment (start 121.740892 106.701) (end 119.138892 104.099) (width 0.2) (layer "F.Cu") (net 11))
 (segment (start 118.357 103.143) (end 98.777 103.143) (width 0.2) (layer "F.Cu") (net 11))
 (segment (start 134.028496 105.038604) (end 134.251 105.261108) (width 0.2) (layer "F.Cu") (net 11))
 (segment (start 134.251 105.261108) (end 134.251 106.338892) (width 0.2) (layer "F.Cu") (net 11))
 (segment (start 118.6 102.9) (end 118.357 103.143) (width 0.2) (layer "F.Cu") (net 11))
 (segment (start 133.488892 107.101) (end 132.411108 107.101) (width 0.2) (layer "F.Cu") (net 11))
 (segment (start 92.408 107.961626) (end 92.408 100.81437) (width 0.2) (layer "F.Cu") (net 10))
 (segment (start 92.408 100.81437) (end 93.68237 99.54) (width 0.2) (layer "F.Cu") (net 10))
 (segment (start 92.669374 108.223) (end 92.408 107.961626) (width 0.2) (layer "F.Cu") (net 10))
 (segment (start 118.6 105.4) (end 115.777 108.223) (width 0.2) (layer "F.Cu") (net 10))
 (segment (start 93.68237 99.54) (end 94.76 99.54) (width 0.2) (layer "F.Cu") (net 10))
 (segment (start 115.777 108.223) (end 92.669374 108.223) (width 0.2) (layer "F.Cu") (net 10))
 (segment (start 129.943 92.797) (end 110.3 92.797) (width 0.2) (layer "F.Cu") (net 15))
 (segment (start 137.025 85.715) (end 129.943 92.797) (width 0.2) (layer "F.Cu") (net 15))
 (via (at 110.3 92.797) (size 0.6) (drill 0.3) (layers "F.Cu" "B.Cu") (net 15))
 (segment (start 109.55969 95.937) (end 108.937 96.55969) (width 0.2) (layer "B.Cu") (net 15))
 (segment (start 108.937 96.55969) (end 108.937 98.477) (width 0.2) (layer "B.Cu") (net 15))
 (segment (start 110.3 92.797) (end 111.063 93.56) (width 0.2) (layer "B.Cu") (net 15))
 (segment (start 111.063 93.56) (end 111.063 95.31431) (width 0.2) (layer "B.Cu") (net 15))
 (segment (start 108.937 98.477) (end 110 99.54) (width 0.2) (layer "B.Cu") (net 15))
 (segment (start 110.44031 95.937) (end 109.55969 95.937) (width 0.2) (layer "B.Cu") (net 15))
 (segment (start 111.063 95.31431) (end 110.44031 95.937) (width 0.2) (layer "B.Cu") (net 15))
 (segment (start 134.423 93.397) (end 92.669374 93.397) (width 0.2) (layer "F.Cu") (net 13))
 (segment (start 92.669374 93.397) (end 92.408 93.658374) (width 0.2) (layer "F.Cu") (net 13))
 (segment (start 95.823 99.09969) (end 95.823 103.557) (width 0.2) (layer "F.Cu") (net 13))
 (segment (start 94.938936 98.215626) (end 95.823 99.09969) (width 0.2) (layer "F.Cu") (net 13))
 (segment (start 142.105 85.715) (end 134.423 93.397) (width 0.2) (layer "F.Cu") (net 13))
 (segment (start 92.408 93.658374) (end 92.408 98.215626) (width 0.2) (layer "F.Cu") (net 13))
 (segment (start 92.408 98.215626) (end 94.938936 98.215626) (width 0.2) (layer "F.Cu") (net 13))
 (segment (start 95.823 103.557) (end 94.76 104.62) (width 0.2) (layer "F.Cu") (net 13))
 (segment (start 143.256 85.23824) (end 143.256 86.19176) (width 0.2) (layer "F.Cu") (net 14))
 (segment (start 142.58176 84.564) (end 143.256 85.23824) (width 0.2) (layer "F.Cu") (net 14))
 (segment (start 134.52476 94.923) (end 113.7 94.923) (width 0.2) (layer "F.Cu") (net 14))
 (segment (start 139.565 85.715) (end 140.716 84.564) (width 0.2) (layer "F.Cu") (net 14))
 (segment (start 140.716 84.564) (end 142.58176 84.564) (width 0.2) (layer "F.Cu") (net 14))
 (segment (start 143.256 86.19176) (end 134.52476 94.923) (width 0.2) (layer "F.Cu") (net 14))
 (via (at 113.7 94.923) (size 0.6) (drill 0.3) (layers "F.Cu" "B.Cu") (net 14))
 (segment (start 113.677 94.923) (end 111.6 97) (width 0.2) (layer "B.Cu") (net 14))
 (segment (start 111.6 97) (end 110 97) (width 0.2) (layer "B.Cu") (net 14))
 (segment (start 113.7 94.923) (end 113.677 94.923) (width 0.2) (layer "B.Cu") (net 14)))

